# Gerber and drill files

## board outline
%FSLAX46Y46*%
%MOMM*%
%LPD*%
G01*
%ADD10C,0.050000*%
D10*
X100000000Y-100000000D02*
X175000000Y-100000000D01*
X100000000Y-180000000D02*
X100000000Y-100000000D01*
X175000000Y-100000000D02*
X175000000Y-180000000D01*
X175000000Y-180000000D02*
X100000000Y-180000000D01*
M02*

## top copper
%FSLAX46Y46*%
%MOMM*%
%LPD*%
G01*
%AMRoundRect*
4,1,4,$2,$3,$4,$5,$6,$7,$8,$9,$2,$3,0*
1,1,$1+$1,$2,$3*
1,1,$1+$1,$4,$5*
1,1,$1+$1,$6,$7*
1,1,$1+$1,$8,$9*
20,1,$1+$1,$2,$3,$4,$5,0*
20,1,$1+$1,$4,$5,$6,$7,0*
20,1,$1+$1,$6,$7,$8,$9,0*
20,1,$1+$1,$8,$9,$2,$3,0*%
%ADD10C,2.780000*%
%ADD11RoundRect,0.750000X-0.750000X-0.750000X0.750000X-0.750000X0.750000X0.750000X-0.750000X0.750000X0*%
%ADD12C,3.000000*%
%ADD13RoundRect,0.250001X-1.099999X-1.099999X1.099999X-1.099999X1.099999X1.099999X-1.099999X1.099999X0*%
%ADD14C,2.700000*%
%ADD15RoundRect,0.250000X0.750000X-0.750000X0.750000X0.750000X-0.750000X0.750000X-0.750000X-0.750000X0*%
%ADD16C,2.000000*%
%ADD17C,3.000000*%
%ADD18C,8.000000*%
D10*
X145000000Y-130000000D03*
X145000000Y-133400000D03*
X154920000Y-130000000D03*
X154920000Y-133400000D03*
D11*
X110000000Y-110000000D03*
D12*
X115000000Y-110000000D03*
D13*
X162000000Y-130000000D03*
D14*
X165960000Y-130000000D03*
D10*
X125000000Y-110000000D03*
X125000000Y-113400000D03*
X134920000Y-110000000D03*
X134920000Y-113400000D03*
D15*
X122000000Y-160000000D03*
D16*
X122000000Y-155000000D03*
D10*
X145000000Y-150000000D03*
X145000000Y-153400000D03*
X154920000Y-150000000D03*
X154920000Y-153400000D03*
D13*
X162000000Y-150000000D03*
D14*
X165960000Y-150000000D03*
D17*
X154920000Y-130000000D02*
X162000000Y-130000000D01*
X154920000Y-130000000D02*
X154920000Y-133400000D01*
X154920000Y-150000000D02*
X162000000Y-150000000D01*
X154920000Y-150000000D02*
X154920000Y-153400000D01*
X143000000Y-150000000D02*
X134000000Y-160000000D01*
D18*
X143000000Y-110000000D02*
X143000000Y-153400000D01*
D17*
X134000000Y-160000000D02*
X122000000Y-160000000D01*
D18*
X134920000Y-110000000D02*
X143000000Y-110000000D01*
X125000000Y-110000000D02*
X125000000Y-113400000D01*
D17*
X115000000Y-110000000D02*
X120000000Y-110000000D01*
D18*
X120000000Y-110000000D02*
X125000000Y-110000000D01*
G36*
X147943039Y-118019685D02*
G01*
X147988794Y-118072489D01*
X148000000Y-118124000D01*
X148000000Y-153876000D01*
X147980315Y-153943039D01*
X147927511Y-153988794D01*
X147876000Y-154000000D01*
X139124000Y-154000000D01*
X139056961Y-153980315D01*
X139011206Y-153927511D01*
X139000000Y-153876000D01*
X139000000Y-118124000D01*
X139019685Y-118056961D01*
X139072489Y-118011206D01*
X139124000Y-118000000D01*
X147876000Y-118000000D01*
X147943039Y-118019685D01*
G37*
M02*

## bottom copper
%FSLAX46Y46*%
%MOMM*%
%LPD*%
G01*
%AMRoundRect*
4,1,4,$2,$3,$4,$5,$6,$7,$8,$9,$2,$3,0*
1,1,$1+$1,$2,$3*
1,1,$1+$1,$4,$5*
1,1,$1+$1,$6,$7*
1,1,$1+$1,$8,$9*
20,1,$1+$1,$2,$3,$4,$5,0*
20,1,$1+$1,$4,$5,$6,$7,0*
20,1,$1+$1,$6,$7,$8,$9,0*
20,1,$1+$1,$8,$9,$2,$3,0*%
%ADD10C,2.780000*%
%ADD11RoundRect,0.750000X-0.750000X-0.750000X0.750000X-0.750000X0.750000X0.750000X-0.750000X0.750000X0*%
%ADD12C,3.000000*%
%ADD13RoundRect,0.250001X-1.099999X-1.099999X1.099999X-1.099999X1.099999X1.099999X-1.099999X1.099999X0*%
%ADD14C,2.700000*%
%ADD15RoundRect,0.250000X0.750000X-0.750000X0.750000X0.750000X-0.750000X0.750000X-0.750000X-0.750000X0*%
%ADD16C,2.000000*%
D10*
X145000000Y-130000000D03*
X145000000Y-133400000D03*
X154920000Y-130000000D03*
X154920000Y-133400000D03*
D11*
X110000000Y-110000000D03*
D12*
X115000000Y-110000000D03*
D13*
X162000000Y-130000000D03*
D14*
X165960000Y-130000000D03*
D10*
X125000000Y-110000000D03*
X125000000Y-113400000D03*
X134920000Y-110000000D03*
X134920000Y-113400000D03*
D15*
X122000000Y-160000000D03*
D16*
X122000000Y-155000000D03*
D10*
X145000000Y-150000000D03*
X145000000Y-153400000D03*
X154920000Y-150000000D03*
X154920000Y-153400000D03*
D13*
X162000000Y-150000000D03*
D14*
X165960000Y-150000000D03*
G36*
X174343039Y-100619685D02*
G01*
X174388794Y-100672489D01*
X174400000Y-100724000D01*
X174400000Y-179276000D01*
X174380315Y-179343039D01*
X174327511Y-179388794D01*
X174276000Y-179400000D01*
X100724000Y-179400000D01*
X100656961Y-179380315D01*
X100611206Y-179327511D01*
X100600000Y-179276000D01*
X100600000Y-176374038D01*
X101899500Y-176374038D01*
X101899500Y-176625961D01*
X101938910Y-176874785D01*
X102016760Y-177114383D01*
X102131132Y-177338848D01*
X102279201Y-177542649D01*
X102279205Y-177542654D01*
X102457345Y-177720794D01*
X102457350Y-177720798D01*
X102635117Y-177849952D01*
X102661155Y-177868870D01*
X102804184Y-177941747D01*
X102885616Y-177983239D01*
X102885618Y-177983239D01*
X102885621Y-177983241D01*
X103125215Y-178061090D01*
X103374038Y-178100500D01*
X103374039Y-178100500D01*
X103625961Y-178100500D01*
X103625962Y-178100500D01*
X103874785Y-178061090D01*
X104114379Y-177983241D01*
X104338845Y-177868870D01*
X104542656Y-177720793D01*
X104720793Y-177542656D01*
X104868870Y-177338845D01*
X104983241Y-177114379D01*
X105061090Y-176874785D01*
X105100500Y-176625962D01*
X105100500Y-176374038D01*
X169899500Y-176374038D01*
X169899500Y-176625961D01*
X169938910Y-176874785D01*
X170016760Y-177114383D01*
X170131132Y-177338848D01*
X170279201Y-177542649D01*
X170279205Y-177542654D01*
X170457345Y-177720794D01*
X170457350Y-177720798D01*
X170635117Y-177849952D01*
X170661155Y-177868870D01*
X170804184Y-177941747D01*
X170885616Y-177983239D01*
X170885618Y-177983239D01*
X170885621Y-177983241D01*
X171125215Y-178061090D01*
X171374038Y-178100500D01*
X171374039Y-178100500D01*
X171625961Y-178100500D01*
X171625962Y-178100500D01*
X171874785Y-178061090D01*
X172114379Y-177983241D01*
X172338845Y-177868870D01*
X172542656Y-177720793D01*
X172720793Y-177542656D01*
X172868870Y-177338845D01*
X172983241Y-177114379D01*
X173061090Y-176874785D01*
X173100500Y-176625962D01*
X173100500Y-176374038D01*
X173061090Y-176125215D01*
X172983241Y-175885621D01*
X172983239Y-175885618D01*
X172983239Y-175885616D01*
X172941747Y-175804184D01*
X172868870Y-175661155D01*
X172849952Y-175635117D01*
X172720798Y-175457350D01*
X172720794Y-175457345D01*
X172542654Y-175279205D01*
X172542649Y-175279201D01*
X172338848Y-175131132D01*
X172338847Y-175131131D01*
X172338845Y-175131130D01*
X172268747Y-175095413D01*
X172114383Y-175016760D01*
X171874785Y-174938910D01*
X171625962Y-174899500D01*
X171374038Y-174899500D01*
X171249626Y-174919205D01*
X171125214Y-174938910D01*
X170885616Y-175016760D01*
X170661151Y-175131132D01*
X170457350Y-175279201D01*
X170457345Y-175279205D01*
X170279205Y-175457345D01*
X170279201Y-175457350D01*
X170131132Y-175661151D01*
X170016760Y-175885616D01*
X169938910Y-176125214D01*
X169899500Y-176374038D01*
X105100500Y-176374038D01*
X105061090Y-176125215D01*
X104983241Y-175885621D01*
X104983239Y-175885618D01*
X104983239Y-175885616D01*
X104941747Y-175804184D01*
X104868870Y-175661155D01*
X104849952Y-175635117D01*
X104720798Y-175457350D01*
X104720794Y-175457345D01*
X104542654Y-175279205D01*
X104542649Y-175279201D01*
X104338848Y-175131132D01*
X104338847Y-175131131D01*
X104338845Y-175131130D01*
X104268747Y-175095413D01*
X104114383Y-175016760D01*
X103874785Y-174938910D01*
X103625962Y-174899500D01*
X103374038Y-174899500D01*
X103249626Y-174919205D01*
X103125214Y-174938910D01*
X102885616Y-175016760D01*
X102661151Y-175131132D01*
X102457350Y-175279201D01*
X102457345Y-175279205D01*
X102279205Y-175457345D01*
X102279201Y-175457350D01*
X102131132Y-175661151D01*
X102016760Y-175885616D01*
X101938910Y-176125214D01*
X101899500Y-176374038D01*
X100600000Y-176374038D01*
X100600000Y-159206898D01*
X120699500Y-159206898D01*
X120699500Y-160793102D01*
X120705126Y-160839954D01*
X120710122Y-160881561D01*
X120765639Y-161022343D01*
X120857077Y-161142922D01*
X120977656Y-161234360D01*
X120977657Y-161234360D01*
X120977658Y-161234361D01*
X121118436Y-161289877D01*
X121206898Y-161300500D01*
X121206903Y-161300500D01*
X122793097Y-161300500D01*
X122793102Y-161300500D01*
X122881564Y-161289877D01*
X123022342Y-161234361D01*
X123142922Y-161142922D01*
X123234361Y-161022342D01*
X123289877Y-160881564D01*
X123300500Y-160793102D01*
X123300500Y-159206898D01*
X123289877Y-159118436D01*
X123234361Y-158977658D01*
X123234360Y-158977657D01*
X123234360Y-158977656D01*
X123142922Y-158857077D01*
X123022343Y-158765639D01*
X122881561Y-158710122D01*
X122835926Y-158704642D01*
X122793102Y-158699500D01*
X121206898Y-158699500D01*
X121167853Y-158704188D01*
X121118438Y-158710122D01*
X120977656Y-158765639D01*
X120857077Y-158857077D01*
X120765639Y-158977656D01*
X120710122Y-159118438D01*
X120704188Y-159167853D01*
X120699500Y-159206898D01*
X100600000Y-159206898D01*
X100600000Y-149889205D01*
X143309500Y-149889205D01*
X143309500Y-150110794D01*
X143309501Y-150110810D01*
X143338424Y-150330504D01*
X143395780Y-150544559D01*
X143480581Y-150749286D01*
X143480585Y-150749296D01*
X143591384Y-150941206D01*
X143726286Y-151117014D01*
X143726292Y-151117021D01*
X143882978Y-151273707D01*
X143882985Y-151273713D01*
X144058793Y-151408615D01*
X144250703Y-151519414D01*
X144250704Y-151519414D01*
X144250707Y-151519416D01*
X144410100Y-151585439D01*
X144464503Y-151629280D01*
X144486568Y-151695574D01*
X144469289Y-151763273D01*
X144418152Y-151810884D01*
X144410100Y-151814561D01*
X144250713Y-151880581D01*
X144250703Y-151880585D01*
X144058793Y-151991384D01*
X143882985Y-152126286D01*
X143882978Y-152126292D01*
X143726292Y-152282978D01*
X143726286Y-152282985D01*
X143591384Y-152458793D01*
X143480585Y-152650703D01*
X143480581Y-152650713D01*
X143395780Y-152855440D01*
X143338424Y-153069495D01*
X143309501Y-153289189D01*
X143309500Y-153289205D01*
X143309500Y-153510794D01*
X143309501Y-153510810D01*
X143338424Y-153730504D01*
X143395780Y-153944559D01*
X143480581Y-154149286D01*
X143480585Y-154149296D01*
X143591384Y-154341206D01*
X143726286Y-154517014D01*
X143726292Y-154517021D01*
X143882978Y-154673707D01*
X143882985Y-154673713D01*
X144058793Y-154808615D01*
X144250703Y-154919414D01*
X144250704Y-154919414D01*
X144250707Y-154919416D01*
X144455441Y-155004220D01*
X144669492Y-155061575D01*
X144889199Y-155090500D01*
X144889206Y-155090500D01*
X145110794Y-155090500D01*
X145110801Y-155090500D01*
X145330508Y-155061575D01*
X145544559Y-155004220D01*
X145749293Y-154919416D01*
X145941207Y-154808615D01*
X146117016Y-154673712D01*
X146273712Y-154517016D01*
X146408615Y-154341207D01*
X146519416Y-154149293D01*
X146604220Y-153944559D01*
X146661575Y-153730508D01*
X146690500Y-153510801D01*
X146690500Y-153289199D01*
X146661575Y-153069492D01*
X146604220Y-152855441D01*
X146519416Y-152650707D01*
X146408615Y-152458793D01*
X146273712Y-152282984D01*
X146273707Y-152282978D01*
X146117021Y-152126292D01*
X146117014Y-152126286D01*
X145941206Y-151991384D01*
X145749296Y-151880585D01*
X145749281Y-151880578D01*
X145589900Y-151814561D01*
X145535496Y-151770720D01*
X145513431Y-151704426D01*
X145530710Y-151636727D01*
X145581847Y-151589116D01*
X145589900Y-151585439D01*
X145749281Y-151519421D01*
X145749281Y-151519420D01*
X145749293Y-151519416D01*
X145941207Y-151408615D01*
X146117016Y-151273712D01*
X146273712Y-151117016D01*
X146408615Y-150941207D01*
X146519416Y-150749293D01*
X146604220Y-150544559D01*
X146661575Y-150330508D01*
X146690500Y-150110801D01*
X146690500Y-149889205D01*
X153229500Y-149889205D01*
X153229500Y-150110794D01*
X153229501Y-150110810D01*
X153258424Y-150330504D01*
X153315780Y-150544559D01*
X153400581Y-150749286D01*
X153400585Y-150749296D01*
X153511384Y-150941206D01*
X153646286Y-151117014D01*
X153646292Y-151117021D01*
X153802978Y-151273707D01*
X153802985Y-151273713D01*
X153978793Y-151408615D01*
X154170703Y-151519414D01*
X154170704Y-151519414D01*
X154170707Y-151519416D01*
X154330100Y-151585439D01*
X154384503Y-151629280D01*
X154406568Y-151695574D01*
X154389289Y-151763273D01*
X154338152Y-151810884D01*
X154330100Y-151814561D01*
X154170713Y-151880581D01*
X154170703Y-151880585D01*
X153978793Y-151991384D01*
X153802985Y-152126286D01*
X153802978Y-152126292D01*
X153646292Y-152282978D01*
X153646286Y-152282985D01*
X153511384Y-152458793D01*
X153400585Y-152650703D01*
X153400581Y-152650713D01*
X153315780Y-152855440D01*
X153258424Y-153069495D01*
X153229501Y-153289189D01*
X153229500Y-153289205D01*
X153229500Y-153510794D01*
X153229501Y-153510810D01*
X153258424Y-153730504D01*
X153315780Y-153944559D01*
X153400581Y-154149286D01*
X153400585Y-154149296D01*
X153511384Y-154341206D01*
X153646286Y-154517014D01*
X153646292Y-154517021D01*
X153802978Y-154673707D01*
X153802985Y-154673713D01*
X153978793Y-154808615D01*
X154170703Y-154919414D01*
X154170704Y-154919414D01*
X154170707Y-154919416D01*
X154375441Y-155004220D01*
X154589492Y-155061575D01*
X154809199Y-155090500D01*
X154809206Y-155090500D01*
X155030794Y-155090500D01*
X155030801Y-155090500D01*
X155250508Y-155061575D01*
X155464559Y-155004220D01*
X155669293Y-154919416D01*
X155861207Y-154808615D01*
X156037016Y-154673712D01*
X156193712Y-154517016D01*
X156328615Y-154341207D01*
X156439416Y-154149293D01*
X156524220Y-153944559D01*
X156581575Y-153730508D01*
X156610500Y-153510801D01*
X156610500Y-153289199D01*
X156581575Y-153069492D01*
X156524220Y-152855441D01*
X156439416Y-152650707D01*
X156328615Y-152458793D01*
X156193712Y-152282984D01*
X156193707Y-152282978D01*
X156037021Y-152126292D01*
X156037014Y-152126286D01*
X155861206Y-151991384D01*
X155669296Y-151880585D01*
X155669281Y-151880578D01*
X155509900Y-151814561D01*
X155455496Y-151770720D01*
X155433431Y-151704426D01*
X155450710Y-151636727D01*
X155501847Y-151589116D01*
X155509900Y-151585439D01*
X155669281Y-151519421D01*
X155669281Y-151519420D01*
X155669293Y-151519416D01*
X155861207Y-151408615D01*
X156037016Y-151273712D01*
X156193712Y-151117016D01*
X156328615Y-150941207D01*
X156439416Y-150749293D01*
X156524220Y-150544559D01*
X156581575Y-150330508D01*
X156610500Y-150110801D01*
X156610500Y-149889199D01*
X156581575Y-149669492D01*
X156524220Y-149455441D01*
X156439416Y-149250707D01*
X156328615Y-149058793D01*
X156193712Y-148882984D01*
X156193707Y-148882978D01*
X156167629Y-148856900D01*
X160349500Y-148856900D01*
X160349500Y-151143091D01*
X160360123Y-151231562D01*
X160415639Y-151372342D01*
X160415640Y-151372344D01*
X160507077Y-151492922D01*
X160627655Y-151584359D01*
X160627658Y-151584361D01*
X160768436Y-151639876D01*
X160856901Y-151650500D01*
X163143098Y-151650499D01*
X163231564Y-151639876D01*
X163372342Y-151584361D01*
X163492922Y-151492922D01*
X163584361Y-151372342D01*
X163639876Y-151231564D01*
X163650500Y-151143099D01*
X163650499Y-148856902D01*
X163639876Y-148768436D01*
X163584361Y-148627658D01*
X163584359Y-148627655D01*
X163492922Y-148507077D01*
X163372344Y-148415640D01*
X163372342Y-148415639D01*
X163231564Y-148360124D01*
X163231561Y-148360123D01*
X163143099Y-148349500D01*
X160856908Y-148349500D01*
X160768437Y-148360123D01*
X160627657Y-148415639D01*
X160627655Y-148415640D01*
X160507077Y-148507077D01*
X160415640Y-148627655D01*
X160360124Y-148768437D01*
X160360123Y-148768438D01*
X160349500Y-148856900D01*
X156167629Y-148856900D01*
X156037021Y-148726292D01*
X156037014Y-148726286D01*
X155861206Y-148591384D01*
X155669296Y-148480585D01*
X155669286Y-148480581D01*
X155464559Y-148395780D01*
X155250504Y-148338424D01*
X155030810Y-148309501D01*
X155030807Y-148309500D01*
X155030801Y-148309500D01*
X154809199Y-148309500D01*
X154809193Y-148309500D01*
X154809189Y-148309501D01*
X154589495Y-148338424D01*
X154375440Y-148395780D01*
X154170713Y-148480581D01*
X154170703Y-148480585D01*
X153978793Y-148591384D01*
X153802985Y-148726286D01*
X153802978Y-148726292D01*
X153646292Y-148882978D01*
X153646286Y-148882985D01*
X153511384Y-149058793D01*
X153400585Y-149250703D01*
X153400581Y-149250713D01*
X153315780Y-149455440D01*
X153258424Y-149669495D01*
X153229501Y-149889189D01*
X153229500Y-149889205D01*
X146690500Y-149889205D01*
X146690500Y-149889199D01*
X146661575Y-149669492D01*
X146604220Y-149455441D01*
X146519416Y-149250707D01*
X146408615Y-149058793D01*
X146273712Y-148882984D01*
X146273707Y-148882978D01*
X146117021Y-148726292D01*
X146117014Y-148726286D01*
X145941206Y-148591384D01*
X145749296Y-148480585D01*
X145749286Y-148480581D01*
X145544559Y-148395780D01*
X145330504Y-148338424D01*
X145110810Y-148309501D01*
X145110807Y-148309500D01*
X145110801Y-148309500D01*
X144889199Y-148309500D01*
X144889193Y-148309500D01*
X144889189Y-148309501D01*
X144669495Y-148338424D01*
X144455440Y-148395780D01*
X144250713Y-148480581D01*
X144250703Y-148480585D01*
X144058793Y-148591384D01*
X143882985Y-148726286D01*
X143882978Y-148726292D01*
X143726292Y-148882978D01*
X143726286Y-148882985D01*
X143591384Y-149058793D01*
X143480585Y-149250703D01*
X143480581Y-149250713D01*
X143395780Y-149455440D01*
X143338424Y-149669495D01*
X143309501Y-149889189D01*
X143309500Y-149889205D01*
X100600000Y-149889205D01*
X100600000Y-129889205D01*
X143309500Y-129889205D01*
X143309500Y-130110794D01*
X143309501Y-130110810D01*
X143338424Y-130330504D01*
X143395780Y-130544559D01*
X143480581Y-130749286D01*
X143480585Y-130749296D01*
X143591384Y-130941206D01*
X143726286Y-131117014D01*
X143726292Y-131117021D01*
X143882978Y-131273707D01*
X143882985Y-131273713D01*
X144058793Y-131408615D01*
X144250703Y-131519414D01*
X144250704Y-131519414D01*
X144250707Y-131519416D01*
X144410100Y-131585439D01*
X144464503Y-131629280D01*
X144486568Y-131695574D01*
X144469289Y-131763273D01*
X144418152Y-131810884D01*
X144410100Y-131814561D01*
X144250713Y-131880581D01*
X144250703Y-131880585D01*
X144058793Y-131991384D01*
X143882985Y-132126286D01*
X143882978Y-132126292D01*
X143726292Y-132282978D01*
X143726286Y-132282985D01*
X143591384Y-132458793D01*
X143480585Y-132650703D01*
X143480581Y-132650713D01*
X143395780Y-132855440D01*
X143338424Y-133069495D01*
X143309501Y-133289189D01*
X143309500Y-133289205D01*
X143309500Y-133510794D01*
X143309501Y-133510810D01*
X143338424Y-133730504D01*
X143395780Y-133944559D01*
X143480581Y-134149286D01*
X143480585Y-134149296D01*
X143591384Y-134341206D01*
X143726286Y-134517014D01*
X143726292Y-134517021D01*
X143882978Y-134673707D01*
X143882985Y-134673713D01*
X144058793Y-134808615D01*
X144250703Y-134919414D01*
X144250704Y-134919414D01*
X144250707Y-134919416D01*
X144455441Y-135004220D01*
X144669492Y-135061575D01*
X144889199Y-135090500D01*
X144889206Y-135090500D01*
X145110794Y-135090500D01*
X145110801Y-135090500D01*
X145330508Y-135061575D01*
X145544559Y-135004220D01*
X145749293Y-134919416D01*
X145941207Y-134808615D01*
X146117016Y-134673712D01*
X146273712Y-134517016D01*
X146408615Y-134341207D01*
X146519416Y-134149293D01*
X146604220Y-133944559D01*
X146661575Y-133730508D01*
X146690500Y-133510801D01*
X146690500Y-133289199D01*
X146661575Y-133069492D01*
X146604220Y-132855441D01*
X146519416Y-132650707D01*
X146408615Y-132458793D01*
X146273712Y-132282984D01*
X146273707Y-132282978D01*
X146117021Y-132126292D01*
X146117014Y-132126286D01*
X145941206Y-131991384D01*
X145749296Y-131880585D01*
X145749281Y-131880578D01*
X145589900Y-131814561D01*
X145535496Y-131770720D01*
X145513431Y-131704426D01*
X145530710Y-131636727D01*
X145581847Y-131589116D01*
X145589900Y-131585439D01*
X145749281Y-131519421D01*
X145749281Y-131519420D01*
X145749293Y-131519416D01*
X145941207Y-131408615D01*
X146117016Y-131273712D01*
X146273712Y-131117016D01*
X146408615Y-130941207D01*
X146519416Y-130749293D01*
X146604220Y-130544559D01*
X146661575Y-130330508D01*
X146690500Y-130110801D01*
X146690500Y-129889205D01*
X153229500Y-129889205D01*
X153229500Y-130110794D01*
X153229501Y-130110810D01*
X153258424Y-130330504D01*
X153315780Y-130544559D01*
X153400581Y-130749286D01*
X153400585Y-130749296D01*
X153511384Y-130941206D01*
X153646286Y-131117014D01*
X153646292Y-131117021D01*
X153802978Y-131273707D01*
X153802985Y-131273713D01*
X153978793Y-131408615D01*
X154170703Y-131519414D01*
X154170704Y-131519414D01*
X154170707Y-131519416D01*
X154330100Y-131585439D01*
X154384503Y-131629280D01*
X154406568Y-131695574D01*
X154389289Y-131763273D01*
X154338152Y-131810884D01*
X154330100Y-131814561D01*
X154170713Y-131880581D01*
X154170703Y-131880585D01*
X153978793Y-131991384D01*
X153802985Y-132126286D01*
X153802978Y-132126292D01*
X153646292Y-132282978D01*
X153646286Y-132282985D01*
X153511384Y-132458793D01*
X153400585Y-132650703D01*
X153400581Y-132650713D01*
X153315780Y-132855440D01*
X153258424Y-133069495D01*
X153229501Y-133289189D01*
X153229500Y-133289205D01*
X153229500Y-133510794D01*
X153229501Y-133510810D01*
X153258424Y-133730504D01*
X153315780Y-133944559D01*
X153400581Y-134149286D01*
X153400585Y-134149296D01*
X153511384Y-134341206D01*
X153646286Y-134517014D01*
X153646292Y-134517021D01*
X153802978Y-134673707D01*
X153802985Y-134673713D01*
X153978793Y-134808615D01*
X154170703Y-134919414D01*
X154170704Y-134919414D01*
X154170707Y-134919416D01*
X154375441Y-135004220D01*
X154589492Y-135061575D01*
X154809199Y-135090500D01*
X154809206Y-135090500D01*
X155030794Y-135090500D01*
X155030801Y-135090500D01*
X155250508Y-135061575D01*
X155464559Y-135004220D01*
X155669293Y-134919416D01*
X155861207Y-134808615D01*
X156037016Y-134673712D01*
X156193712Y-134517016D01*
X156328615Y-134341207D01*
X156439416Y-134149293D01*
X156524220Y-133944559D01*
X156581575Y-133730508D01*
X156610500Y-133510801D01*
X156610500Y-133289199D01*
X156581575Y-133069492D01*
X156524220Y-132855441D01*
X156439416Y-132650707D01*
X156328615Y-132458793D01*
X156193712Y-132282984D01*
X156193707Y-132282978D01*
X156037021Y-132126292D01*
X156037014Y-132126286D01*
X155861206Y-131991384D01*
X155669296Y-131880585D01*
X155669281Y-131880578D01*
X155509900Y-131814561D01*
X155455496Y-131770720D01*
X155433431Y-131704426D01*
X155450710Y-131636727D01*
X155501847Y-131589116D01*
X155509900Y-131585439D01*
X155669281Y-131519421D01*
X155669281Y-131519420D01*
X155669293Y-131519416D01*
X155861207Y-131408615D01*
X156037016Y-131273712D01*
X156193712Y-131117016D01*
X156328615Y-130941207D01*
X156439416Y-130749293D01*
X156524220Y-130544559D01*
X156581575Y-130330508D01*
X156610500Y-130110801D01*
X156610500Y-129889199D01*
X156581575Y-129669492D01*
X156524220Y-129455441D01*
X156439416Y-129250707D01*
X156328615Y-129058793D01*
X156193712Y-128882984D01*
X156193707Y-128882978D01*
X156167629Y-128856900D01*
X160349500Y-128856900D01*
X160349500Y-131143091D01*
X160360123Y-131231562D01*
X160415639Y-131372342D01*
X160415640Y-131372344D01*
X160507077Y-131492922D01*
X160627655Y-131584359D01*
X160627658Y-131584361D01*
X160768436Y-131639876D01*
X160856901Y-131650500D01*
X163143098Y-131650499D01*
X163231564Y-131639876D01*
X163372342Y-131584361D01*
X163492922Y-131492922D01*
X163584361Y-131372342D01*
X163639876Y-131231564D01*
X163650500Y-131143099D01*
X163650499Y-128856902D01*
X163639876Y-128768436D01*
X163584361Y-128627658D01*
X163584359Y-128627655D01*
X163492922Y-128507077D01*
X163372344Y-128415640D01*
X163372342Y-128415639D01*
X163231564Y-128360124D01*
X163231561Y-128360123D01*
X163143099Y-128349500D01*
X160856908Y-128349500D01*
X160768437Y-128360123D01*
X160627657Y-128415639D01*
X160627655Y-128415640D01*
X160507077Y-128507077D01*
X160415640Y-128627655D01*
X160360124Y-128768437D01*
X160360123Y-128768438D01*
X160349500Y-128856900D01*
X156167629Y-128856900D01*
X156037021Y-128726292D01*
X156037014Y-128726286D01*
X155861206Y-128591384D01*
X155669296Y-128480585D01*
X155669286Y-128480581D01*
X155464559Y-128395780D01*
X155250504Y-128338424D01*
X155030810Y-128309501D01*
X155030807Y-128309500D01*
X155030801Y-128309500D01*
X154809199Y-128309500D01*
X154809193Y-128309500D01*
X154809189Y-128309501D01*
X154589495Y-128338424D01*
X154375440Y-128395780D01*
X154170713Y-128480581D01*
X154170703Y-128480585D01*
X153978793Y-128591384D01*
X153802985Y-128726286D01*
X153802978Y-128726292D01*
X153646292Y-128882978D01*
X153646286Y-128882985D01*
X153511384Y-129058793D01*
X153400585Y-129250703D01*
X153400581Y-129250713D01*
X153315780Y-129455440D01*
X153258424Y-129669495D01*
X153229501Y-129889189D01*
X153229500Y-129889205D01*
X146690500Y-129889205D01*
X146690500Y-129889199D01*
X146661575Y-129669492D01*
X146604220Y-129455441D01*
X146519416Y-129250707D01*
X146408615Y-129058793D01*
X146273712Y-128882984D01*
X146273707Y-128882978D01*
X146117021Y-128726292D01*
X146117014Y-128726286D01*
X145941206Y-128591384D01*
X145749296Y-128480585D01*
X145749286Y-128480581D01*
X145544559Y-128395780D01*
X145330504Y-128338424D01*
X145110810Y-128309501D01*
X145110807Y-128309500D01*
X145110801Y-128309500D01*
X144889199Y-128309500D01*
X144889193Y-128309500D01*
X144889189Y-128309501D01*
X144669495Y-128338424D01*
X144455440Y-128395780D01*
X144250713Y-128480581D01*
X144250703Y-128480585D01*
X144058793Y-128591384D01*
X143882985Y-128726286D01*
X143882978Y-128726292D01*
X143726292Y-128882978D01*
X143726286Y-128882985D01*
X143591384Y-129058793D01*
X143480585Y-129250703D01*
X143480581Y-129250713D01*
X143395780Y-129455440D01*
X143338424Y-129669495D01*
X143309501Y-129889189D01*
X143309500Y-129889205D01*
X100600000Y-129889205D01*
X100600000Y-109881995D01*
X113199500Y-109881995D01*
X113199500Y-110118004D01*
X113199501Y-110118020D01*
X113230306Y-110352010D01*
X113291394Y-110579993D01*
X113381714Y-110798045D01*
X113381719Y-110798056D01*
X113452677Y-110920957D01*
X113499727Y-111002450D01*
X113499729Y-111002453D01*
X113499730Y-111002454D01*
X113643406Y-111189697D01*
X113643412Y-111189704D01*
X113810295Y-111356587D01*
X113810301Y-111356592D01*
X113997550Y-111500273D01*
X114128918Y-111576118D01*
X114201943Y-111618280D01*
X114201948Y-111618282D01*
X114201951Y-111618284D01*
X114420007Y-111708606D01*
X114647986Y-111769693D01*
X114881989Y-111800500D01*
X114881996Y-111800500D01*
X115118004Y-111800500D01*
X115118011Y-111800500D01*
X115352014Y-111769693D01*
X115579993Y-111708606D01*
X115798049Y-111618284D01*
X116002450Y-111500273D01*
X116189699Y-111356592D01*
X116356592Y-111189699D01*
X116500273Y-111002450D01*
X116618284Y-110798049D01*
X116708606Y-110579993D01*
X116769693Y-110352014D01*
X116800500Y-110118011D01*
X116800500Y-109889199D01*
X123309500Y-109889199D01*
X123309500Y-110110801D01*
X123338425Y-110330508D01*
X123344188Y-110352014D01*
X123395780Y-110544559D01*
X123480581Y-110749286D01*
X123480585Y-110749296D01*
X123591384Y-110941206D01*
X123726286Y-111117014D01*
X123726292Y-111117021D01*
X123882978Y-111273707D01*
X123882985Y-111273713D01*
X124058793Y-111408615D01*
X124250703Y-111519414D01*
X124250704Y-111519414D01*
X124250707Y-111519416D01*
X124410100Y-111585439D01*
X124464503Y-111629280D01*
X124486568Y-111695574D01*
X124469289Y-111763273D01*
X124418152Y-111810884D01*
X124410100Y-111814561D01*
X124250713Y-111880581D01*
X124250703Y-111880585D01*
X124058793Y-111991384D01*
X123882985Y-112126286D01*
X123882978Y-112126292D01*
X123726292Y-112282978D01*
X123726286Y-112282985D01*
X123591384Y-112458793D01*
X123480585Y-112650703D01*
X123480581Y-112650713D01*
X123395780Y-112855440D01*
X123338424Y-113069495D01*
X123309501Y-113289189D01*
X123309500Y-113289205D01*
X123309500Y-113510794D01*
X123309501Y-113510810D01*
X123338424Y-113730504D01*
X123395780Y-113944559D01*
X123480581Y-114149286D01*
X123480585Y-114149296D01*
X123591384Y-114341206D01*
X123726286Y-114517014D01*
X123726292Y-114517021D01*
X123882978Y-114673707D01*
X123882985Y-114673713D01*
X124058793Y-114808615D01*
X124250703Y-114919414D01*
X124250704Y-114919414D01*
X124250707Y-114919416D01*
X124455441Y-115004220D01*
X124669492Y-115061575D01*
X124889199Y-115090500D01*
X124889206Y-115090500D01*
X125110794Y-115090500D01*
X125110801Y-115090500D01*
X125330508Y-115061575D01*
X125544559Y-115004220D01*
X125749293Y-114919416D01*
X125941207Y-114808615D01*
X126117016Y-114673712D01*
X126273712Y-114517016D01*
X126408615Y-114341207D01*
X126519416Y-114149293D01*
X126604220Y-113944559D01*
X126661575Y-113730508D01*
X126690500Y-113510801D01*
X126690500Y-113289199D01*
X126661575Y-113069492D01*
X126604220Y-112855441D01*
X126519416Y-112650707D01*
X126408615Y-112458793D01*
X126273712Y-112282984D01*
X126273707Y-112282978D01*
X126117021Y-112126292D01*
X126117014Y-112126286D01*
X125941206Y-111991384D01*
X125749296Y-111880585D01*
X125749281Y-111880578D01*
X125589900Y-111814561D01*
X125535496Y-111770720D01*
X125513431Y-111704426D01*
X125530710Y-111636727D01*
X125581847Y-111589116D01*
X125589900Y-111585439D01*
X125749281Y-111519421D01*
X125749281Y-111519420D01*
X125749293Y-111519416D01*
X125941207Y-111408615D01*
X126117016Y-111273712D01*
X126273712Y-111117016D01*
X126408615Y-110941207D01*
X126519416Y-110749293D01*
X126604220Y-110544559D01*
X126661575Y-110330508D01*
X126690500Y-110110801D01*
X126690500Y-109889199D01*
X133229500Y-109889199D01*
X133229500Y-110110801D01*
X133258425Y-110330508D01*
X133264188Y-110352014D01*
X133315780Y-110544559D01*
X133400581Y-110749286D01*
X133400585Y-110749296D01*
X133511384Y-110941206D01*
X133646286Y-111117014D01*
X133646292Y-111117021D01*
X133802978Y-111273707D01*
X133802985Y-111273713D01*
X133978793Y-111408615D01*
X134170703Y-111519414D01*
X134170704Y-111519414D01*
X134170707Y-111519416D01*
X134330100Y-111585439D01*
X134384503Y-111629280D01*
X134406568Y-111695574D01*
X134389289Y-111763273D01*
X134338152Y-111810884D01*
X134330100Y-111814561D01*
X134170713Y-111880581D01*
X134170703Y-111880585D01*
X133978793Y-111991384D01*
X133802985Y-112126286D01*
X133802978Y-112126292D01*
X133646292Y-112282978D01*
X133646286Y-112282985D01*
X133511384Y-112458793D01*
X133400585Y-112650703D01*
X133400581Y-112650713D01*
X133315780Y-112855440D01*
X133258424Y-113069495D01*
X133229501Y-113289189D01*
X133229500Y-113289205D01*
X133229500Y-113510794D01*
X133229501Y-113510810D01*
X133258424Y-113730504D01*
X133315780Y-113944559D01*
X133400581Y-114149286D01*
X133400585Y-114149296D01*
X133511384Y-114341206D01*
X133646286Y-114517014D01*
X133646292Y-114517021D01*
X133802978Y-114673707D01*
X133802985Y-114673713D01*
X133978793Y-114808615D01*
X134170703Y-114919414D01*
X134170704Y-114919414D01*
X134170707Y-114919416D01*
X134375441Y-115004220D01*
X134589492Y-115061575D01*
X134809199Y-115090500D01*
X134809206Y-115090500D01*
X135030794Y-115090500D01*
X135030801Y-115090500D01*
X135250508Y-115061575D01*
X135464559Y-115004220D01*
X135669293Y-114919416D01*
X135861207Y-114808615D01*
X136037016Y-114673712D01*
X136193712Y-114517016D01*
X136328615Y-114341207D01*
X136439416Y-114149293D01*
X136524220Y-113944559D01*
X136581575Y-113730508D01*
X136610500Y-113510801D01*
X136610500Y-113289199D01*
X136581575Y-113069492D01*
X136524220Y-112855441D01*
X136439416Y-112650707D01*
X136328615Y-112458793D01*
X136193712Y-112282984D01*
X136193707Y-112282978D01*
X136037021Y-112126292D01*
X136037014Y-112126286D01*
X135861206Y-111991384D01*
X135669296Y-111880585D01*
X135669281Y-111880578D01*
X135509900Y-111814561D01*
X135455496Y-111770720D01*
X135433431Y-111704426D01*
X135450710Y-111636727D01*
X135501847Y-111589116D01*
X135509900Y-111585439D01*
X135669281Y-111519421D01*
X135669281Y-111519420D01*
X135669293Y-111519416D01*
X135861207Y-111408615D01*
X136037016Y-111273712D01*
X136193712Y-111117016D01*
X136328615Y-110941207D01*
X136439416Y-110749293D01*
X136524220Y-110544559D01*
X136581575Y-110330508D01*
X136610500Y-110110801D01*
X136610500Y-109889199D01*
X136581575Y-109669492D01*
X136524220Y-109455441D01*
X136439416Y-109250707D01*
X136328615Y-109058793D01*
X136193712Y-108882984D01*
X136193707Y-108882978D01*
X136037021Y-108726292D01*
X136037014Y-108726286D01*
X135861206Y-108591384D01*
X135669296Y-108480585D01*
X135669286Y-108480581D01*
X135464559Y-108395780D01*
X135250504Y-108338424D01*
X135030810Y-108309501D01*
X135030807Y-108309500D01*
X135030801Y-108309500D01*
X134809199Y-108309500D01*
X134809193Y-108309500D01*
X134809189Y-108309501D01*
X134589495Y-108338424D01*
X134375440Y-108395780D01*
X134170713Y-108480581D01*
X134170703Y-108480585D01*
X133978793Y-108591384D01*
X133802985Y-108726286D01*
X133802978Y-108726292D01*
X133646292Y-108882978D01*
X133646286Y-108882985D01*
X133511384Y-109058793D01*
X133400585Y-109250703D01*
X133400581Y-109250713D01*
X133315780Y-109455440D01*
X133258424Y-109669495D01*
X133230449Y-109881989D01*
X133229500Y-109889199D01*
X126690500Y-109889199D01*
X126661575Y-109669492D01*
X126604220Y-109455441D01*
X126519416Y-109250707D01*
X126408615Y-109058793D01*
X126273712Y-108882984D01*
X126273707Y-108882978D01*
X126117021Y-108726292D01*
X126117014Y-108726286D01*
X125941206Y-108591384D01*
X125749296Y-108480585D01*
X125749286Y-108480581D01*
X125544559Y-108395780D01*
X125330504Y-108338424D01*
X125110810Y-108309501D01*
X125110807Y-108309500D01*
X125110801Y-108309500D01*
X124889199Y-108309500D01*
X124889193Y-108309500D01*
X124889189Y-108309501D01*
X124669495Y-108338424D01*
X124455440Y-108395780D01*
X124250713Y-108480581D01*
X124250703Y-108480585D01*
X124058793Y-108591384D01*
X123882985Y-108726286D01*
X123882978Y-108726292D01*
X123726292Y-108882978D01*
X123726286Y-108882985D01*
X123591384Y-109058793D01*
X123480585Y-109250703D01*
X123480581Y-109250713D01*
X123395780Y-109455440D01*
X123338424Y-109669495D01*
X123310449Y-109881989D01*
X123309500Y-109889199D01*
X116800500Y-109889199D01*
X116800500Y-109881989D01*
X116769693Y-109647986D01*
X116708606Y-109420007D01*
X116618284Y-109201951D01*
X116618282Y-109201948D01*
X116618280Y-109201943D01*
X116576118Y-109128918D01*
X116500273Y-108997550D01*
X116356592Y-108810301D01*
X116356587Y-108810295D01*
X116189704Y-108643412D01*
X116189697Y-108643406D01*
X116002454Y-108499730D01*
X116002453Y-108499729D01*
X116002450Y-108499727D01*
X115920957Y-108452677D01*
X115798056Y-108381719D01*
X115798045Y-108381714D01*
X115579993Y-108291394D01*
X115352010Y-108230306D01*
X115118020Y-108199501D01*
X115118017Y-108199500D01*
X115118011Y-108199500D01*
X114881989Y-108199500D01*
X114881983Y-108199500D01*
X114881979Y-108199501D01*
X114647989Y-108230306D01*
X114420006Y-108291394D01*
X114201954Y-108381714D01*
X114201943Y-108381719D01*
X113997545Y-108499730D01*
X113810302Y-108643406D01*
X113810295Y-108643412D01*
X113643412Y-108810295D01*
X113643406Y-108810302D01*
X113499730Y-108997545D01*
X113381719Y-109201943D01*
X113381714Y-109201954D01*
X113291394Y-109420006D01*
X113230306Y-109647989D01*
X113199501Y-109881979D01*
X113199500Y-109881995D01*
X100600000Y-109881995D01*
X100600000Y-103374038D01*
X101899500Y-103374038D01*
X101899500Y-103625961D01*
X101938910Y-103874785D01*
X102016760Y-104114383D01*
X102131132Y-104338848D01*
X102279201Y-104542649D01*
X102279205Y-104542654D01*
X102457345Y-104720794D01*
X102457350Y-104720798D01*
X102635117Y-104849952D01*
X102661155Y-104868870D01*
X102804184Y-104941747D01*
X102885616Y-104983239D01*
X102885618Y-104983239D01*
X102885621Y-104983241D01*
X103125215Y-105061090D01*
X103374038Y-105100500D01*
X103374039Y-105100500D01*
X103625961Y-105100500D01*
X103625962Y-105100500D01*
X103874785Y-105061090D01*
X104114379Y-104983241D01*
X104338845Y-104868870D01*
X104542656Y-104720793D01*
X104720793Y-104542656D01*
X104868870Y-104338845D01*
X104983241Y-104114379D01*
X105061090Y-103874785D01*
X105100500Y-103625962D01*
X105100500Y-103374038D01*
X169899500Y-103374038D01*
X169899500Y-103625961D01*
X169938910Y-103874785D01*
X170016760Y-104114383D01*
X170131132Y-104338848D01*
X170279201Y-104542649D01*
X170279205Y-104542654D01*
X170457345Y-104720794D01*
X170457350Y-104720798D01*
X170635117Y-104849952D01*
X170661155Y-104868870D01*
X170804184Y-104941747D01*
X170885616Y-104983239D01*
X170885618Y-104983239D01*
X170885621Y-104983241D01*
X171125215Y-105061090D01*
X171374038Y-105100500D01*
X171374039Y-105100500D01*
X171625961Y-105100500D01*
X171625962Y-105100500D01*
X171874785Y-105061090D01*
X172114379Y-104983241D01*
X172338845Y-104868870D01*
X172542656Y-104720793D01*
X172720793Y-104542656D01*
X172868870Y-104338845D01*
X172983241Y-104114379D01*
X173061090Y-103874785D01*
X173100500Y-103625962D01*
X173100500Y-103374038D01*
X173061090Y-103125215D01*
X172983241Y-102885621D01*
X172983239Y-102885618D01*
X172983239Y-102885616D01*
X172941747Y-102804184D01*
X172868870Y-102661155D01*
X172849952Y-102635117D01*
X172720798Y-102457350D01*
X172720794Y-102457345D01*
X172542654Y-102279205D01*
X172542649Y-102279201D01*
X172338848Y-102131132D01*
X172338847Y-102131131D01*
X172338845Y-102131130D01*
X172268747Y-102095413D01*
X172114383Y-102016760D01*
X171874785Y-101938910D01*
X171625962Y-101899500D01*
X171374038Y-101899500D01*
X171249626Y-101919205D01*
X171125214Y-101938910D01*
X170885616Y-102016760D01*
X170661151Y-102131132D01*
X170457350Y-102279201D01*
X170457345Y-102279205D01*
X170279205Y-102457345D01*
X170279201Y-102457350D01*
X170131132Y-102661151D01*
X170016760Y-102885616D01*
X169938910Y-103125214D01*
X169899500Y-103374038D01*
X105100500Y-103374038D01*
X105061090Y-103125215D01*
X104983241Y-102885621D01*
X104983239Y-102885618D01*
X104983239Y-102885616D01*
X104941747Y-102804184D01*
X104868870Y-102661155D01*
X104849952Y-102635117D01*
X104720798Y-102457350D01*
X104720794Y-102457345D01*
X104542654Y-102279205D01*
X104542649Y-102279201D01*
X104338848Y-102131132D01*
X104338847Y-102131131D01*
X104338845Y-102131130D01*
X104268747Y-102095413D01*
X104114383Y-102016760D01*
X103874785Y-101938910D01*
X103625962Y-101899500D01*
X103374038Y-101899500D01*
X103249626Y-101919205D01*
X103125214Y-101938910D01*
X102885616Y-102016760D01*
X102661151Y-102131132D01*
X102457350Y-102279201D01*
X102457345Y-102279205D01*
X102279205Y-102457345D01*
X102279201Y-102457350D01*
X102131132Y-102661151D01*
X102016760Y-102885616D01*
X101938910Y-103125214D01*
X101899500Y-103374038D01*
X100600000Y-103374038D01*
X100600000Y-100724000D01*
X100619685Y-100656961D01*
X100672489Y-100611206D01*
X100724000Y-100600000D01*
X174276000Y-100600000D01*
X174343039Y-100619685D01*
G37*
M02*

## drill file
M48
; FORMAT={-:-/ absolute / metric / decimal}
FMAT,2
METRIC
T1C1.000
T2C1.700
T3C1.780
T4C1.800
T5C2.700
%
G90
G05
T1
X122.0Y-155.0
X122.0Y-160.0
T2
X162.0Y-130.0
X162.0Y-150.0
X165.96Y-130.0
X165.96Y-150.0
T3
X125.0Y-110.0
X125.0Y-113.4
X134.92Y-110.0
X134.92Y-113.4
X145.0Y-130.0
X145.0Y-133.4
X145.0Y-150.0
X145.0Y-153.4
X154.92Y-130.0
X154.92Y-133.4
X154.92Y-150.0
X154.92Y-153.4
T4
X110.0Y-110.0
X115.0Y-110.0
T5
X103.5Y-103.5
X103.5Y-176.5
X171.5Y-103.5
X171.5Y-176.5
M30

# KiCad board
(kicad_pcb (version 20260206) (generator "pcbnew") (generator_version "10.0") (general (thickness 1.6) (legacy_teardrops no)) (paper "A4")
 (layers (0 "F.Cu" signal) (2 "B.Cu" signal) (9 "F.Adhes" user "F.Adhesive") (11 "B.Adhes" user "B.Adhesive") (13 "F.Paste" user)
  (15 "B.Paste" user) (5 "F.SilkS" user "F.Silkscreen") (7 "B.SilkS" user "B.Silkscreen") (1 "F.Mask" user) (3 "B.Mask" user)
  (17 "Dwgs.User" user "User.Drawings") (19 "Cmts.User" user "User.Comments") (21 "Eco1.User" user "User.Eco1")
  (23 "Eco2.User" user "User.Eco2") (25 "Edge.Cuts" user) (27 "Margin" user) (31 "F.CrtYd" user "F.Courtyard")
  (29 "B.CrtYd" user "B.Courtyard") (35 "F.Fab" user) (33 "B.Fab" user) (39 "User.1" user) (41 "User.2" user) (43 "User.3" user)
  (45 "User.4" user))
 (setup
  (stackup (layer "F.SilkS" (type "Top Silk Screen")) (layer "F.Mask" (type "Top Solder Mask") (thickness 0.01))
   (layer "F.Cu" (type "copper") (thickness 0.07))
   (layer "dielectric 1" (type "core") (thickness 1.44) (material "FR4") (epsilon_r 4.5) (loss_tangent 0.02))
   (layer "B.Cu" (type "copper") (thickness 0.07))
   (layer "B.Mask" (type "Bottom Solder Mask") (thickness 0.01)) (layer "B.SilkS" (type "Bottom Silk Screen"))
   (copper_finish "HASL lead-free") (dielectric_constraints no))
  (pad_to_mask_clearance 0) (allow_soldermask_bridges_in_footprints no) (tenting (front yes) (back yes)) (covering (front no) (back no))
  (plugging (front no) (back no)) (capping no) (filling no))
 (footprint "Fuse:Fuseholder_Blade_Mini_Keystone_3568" (layer "F.Cu") (at 145 130)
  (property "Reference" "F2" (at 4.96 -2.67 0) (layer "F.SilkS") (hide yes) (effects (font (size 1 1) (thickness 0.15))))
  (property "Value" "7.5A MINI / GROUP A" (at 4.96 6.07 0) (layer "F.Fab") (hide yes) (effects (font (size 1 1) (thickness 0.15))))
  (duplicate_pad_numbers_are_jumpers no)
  (pad "1" thru_hole circle (at 0 0) (size 2.78 2.78) (drill 1.78) (layers "*.Cu" "*.Mask") (remove_unused_layers no) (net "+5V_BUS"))
  (pad "1" thru_hole circle (at 0 3.4) (size 2.78 2.78) (drill 1.78) (layers "*.Cu" "*.Mask") (remove_unused_layers no) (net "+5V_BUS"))
  (pad "2" thru_hole circle (at 9.92 0) (size 2.78 2.78) (drill 1.78) (layers "*.Cu" "*.Mask") (remove_unused_layers no) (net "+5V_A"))
  (pad "2" thru_hole circle (at 9.92 3.4) (size 2.78 2.78) (drill 1.78) (layers "*.Cu" "*.Mask") (remove_unused_layers no) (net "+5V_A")))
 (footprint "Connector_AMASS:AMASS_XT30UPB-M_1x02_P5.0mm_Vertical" (layer "F.Cu") (at 110 110)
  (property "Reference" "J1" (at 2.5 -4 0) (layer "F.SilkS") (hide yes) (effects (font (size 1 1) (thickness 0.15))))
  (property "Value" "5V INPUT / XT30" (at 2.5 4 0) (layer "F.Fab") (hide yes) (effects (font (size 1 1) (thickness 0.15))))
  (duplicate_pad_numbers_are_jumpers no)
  (pad "1" thru_hole roundrect (at 0 0) (size 3 3) (drill 1.8) (layers "*.Cu" "*.Mask") (remove_unused_layers no) (roundrect_rratio 0.25)
   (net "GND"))
  (pad "2" thru_hole circle (at 5 0) (size 3 3) (drill 1.8) (layers "*.Cu" "*.Mask") (remove_unused_layers no) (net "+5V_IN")))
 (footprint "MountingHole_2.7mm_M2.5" (layer "F.Cu") (at 171.5 176.5)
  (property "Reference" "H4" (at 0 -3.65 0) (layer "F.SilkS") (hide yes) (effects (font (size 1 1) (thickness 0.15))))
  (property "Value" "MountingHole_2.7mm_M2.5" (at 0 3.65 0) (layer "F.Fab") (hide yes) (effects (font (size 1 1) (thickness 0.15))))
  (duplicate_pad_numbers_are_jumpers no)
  (pad "" np_thru_hole circle (at 0 0) (size 2.7 2.7) (drill 2.7) (layers "*.Cu" "*.Mask")))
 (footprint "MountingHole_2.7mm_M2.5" (layer "F.Cu") (at 171.5 103.5)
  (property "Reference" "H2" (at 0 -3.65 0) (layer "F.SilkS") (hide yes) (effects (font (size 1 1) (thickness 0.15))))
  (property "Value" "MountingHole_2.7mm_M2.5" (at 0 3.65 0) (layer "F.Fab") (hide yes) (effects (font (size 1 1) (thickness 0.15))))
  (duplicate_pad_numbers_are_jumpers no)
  (pad "" np_thru_hole circle (at 0 0) (size 2.7 2.7) (drill 2.7) (layers "*.Cu" "*.Mask")))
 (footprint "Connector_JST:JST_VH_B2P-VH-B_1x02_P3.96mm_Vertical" (layer "F.Cu") (at 162 130)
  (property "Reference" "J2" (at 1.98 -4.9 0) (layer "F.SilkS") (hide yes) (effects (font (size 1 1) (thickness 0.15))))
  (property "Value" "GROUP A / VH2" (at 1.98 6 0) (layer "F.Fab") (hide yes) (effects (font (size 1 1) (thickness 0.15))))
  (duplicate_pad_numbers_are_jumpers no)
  (pad "1" thru_hole roundrect (at 0 0) (size 2.7 2.7) (drill 1.7) (layers "*.Cu" "*.Mask") (remove_unused_layers no)
   (roundrect_rratio 0.092593) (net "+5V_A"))
  (pad "2" thru_hole circle (at 3.96 0) (size 2.7 2.7) (drill 1.7) (layers "*.Cu" "*.Mask") (remove_unused_layers no) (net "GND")))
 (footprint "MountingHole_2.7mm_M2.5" (layer "F.Cu") (at 103.5 103.5)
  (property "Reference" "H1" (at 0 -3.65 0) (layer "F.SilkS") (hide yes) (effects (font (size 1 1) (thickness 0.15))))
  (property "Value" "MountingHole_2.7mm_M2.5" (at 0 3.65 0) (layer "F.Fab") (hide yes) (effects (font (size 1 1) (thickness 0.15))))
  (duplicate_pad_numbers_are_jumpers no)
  (pad "" np_thru_hole circle (at 0 0) (size 2.7 2.7) (drill 2.7) (layers "*.Cu" "*.Mask")))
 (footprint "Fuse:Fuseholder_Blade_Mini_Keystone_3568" (layer "F.Cu") (at 125 110)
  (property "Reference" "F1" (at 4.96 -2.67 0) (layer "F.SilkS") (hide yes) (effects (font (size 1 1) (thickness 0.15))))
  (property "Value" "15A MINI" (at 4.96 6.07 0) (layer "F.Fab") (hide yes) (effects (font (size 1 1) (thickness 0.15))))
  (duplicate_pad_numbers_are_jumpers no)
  (pad "1" thru_hole circle (at 0 0) (size 2.78 2.78) (drill 1.78) (layers "*.Cu" "*.Mask") (remove_unused_layers no) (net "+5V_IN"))
  (pad "1" thru_hole circle (at 0 3.4) (size 2.78 2.78) (drill 1.78) (layers "*.Cu" "*.Mask") (remove_unused_layers no) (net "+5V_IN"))
  (pad "2" thru_hole circle (at 9.92 0) (size 2.78 2.78) (drill 1.78) (layers "*.Cu" "*.Mask") (remove_unused_layers no) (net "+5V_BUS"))
  (pad "2" thru_hole circle (at 9.92 3.4) (size 2.78 2.78) (drill 1.78) (layers "*.Cu" "*.Mask") (remove_unused_layers no) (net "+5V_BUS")))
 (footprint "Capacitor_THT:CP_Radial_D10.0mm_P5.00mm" (layer "F.Cu") (at 122 160 90)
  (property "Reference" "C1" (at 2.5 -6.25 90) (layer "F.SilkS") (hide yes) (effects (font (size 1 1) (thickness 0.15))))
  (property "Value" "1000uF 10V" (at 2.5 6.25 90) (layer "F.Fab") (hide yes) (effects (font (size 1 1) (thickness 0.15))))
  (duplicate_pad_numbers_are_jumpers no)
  (pad "1" thru_hole roundrect (at 0 0 90) (size 2 2) (drill 1) (layers "*.Cu" "*.Mask") (remove_unused_layers no) (roundrect_rratio 0.125)
   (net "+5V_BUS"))
  (pad "2" thru_hole circle (at 5 0 90) (size 2 2) (drill 1) (layers "*.Cu" "*.Mask") (remove_unused_layers no) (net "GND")))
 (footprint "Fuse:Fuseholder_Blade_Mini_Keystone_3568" (layer "F.Cu") (at 145 150)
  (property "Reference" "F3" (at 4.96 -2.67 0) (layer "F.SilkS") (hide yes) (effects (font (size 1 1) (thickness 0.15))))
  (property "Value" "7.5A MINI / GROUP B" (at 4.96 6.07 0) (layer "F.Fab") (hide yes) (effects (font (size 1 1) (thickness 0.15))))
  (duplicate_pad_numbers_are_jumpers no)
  (pad "1" thru_hole circle (at 0 0) (size 2.78 2.78) (drill 1.78) (layers "*.Cu" "*.Mask") (remove_unused_layers no) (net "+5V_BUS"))
  (pad "1" thru_hole circle (at 0 3.4) (size 2.78 2.78) (drill 1.78) (layers "*.Cu" "*.Mask") (remove_unused_layers no) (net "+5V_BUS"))
  (pad "2" thru_hole circle (at 9.92 0) (size 2.78 2.78) (drill 1.78) (layers "*.Cu" "*.Mask") (remove_unused_layers no) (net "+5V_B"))
  (pad "2" thru_hole circle (at 9.92 3.4) (size 2.78 2.78) (drill 1.78) (layers "*.Cu" "*.Mask") (remove_unused_layers no) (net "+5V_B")))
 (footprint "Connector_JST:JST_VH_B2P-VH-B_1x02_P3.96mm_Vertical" (layer "F.Cu") (at 162 150)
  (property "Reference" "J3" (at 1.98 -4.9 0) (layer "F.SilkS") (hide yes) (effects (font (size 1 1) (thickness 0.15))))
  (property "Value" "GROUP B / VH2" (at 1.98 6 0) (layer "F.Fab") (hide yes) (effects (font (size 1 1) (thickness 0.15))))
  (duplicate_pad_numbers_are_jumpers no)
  (pad "1" thru_hole roundrect (at 0 0) (size 2.7 2.7) (drill 1.7) (layers "*.Cu" "*.Mask") (remove_unused_layers no)
   (roundrect_rratio 0.092593) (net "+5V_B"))
  (pad "2" thru_hole circle (at 3.96 0) (size 2.7 2.7) (drill 1.7) (layers "*.Cu" "*.Mask") (remove_unused_layers no) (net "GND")))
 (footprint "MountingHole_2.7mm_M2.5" (layer "F.Cu") (at 103.5 176.5)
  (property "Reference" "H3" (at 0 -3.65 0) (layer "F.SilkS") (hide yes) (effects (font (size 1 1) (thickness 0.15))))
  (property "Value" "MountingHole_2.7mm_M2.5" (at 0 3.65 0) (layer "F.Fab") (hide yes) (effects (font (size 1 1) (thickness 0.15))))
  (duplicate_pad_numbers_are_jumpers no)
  (pad "" np_thru_hole circle (at 0 0) (size 2.7 2.7) (drill 2.7) (layers "*.Cu" "*.Mask")))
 (gr_line (start 100 100) (end 175 100) (stroke (width 0.05) (type default)) (layer "Edge.Cuts"))
 (gr_line (start 100 180) (end 100 100) (stroke (width 0.05) (type default)) (layer "Edge.Cuts"))
 (gr_line (start 175 100) (end 175 180) (stroke (width 0.05) (type default)) (layer "Edge.Cuts"))
 (gr_line (start 175 180) (end 100 180) (stroke (width 0.05) (type default)) (layer "Edge.Cuts"))
 (segment (start 154.92 130) (end 162 130) (width 3) (layer "F.Cu") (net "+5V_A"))
 (segment (start 154.92 130) (end 154.92 133.4) (width 3) (layer "F.Cu") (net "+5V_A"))
 (segment (start 154.92 150) (end 162 150) (width 3) (layer "F.Cu") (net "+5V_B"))
 (segment (start 154.92 150) (end 154.92 153.4) (width 3) (layer "F.Cu") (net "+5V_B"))
 (segment (start 143 150) (end 134 160) (width 3) (layer "F.Cu") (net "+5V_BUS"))
 (segment (start 143 110) (end 143 153.4) (width 8) (layer "F.Cu") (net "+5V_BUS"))
 (segment (start 134 160) (end 122 160) (width 3) (layer "F.Cu") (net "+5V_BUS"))
 (segment (start 134.92 110) (end 143 110) (width 8) (layer "F.Cu") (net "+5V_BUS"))
 (segment (start 125 110) (end 125 113.4) (width 8) (layer "F.Cu") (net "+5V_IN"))
 (segment (start 115 110) (end 120 110) (width 3) (layer "F.Cu") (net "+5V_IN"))
 (segment (start 120 110) (end 125 110) (width 8) (layer "F.Cu") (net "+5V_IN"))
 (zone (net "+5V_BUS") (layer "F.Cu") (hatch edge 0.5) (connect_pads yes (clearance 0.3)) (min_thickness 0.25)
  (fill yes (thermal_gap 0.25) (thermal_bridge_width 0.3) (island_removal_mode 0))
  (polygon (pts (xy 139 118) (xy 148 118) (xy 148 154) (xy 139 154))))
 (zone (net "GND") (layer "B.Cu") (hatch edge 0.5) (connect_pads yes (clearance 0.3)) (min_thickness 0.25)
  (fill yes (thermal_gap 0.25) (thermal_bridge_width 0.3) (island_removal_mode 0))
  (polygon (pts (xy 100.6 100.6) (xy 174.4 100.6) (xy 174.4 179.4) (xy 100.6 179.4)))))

